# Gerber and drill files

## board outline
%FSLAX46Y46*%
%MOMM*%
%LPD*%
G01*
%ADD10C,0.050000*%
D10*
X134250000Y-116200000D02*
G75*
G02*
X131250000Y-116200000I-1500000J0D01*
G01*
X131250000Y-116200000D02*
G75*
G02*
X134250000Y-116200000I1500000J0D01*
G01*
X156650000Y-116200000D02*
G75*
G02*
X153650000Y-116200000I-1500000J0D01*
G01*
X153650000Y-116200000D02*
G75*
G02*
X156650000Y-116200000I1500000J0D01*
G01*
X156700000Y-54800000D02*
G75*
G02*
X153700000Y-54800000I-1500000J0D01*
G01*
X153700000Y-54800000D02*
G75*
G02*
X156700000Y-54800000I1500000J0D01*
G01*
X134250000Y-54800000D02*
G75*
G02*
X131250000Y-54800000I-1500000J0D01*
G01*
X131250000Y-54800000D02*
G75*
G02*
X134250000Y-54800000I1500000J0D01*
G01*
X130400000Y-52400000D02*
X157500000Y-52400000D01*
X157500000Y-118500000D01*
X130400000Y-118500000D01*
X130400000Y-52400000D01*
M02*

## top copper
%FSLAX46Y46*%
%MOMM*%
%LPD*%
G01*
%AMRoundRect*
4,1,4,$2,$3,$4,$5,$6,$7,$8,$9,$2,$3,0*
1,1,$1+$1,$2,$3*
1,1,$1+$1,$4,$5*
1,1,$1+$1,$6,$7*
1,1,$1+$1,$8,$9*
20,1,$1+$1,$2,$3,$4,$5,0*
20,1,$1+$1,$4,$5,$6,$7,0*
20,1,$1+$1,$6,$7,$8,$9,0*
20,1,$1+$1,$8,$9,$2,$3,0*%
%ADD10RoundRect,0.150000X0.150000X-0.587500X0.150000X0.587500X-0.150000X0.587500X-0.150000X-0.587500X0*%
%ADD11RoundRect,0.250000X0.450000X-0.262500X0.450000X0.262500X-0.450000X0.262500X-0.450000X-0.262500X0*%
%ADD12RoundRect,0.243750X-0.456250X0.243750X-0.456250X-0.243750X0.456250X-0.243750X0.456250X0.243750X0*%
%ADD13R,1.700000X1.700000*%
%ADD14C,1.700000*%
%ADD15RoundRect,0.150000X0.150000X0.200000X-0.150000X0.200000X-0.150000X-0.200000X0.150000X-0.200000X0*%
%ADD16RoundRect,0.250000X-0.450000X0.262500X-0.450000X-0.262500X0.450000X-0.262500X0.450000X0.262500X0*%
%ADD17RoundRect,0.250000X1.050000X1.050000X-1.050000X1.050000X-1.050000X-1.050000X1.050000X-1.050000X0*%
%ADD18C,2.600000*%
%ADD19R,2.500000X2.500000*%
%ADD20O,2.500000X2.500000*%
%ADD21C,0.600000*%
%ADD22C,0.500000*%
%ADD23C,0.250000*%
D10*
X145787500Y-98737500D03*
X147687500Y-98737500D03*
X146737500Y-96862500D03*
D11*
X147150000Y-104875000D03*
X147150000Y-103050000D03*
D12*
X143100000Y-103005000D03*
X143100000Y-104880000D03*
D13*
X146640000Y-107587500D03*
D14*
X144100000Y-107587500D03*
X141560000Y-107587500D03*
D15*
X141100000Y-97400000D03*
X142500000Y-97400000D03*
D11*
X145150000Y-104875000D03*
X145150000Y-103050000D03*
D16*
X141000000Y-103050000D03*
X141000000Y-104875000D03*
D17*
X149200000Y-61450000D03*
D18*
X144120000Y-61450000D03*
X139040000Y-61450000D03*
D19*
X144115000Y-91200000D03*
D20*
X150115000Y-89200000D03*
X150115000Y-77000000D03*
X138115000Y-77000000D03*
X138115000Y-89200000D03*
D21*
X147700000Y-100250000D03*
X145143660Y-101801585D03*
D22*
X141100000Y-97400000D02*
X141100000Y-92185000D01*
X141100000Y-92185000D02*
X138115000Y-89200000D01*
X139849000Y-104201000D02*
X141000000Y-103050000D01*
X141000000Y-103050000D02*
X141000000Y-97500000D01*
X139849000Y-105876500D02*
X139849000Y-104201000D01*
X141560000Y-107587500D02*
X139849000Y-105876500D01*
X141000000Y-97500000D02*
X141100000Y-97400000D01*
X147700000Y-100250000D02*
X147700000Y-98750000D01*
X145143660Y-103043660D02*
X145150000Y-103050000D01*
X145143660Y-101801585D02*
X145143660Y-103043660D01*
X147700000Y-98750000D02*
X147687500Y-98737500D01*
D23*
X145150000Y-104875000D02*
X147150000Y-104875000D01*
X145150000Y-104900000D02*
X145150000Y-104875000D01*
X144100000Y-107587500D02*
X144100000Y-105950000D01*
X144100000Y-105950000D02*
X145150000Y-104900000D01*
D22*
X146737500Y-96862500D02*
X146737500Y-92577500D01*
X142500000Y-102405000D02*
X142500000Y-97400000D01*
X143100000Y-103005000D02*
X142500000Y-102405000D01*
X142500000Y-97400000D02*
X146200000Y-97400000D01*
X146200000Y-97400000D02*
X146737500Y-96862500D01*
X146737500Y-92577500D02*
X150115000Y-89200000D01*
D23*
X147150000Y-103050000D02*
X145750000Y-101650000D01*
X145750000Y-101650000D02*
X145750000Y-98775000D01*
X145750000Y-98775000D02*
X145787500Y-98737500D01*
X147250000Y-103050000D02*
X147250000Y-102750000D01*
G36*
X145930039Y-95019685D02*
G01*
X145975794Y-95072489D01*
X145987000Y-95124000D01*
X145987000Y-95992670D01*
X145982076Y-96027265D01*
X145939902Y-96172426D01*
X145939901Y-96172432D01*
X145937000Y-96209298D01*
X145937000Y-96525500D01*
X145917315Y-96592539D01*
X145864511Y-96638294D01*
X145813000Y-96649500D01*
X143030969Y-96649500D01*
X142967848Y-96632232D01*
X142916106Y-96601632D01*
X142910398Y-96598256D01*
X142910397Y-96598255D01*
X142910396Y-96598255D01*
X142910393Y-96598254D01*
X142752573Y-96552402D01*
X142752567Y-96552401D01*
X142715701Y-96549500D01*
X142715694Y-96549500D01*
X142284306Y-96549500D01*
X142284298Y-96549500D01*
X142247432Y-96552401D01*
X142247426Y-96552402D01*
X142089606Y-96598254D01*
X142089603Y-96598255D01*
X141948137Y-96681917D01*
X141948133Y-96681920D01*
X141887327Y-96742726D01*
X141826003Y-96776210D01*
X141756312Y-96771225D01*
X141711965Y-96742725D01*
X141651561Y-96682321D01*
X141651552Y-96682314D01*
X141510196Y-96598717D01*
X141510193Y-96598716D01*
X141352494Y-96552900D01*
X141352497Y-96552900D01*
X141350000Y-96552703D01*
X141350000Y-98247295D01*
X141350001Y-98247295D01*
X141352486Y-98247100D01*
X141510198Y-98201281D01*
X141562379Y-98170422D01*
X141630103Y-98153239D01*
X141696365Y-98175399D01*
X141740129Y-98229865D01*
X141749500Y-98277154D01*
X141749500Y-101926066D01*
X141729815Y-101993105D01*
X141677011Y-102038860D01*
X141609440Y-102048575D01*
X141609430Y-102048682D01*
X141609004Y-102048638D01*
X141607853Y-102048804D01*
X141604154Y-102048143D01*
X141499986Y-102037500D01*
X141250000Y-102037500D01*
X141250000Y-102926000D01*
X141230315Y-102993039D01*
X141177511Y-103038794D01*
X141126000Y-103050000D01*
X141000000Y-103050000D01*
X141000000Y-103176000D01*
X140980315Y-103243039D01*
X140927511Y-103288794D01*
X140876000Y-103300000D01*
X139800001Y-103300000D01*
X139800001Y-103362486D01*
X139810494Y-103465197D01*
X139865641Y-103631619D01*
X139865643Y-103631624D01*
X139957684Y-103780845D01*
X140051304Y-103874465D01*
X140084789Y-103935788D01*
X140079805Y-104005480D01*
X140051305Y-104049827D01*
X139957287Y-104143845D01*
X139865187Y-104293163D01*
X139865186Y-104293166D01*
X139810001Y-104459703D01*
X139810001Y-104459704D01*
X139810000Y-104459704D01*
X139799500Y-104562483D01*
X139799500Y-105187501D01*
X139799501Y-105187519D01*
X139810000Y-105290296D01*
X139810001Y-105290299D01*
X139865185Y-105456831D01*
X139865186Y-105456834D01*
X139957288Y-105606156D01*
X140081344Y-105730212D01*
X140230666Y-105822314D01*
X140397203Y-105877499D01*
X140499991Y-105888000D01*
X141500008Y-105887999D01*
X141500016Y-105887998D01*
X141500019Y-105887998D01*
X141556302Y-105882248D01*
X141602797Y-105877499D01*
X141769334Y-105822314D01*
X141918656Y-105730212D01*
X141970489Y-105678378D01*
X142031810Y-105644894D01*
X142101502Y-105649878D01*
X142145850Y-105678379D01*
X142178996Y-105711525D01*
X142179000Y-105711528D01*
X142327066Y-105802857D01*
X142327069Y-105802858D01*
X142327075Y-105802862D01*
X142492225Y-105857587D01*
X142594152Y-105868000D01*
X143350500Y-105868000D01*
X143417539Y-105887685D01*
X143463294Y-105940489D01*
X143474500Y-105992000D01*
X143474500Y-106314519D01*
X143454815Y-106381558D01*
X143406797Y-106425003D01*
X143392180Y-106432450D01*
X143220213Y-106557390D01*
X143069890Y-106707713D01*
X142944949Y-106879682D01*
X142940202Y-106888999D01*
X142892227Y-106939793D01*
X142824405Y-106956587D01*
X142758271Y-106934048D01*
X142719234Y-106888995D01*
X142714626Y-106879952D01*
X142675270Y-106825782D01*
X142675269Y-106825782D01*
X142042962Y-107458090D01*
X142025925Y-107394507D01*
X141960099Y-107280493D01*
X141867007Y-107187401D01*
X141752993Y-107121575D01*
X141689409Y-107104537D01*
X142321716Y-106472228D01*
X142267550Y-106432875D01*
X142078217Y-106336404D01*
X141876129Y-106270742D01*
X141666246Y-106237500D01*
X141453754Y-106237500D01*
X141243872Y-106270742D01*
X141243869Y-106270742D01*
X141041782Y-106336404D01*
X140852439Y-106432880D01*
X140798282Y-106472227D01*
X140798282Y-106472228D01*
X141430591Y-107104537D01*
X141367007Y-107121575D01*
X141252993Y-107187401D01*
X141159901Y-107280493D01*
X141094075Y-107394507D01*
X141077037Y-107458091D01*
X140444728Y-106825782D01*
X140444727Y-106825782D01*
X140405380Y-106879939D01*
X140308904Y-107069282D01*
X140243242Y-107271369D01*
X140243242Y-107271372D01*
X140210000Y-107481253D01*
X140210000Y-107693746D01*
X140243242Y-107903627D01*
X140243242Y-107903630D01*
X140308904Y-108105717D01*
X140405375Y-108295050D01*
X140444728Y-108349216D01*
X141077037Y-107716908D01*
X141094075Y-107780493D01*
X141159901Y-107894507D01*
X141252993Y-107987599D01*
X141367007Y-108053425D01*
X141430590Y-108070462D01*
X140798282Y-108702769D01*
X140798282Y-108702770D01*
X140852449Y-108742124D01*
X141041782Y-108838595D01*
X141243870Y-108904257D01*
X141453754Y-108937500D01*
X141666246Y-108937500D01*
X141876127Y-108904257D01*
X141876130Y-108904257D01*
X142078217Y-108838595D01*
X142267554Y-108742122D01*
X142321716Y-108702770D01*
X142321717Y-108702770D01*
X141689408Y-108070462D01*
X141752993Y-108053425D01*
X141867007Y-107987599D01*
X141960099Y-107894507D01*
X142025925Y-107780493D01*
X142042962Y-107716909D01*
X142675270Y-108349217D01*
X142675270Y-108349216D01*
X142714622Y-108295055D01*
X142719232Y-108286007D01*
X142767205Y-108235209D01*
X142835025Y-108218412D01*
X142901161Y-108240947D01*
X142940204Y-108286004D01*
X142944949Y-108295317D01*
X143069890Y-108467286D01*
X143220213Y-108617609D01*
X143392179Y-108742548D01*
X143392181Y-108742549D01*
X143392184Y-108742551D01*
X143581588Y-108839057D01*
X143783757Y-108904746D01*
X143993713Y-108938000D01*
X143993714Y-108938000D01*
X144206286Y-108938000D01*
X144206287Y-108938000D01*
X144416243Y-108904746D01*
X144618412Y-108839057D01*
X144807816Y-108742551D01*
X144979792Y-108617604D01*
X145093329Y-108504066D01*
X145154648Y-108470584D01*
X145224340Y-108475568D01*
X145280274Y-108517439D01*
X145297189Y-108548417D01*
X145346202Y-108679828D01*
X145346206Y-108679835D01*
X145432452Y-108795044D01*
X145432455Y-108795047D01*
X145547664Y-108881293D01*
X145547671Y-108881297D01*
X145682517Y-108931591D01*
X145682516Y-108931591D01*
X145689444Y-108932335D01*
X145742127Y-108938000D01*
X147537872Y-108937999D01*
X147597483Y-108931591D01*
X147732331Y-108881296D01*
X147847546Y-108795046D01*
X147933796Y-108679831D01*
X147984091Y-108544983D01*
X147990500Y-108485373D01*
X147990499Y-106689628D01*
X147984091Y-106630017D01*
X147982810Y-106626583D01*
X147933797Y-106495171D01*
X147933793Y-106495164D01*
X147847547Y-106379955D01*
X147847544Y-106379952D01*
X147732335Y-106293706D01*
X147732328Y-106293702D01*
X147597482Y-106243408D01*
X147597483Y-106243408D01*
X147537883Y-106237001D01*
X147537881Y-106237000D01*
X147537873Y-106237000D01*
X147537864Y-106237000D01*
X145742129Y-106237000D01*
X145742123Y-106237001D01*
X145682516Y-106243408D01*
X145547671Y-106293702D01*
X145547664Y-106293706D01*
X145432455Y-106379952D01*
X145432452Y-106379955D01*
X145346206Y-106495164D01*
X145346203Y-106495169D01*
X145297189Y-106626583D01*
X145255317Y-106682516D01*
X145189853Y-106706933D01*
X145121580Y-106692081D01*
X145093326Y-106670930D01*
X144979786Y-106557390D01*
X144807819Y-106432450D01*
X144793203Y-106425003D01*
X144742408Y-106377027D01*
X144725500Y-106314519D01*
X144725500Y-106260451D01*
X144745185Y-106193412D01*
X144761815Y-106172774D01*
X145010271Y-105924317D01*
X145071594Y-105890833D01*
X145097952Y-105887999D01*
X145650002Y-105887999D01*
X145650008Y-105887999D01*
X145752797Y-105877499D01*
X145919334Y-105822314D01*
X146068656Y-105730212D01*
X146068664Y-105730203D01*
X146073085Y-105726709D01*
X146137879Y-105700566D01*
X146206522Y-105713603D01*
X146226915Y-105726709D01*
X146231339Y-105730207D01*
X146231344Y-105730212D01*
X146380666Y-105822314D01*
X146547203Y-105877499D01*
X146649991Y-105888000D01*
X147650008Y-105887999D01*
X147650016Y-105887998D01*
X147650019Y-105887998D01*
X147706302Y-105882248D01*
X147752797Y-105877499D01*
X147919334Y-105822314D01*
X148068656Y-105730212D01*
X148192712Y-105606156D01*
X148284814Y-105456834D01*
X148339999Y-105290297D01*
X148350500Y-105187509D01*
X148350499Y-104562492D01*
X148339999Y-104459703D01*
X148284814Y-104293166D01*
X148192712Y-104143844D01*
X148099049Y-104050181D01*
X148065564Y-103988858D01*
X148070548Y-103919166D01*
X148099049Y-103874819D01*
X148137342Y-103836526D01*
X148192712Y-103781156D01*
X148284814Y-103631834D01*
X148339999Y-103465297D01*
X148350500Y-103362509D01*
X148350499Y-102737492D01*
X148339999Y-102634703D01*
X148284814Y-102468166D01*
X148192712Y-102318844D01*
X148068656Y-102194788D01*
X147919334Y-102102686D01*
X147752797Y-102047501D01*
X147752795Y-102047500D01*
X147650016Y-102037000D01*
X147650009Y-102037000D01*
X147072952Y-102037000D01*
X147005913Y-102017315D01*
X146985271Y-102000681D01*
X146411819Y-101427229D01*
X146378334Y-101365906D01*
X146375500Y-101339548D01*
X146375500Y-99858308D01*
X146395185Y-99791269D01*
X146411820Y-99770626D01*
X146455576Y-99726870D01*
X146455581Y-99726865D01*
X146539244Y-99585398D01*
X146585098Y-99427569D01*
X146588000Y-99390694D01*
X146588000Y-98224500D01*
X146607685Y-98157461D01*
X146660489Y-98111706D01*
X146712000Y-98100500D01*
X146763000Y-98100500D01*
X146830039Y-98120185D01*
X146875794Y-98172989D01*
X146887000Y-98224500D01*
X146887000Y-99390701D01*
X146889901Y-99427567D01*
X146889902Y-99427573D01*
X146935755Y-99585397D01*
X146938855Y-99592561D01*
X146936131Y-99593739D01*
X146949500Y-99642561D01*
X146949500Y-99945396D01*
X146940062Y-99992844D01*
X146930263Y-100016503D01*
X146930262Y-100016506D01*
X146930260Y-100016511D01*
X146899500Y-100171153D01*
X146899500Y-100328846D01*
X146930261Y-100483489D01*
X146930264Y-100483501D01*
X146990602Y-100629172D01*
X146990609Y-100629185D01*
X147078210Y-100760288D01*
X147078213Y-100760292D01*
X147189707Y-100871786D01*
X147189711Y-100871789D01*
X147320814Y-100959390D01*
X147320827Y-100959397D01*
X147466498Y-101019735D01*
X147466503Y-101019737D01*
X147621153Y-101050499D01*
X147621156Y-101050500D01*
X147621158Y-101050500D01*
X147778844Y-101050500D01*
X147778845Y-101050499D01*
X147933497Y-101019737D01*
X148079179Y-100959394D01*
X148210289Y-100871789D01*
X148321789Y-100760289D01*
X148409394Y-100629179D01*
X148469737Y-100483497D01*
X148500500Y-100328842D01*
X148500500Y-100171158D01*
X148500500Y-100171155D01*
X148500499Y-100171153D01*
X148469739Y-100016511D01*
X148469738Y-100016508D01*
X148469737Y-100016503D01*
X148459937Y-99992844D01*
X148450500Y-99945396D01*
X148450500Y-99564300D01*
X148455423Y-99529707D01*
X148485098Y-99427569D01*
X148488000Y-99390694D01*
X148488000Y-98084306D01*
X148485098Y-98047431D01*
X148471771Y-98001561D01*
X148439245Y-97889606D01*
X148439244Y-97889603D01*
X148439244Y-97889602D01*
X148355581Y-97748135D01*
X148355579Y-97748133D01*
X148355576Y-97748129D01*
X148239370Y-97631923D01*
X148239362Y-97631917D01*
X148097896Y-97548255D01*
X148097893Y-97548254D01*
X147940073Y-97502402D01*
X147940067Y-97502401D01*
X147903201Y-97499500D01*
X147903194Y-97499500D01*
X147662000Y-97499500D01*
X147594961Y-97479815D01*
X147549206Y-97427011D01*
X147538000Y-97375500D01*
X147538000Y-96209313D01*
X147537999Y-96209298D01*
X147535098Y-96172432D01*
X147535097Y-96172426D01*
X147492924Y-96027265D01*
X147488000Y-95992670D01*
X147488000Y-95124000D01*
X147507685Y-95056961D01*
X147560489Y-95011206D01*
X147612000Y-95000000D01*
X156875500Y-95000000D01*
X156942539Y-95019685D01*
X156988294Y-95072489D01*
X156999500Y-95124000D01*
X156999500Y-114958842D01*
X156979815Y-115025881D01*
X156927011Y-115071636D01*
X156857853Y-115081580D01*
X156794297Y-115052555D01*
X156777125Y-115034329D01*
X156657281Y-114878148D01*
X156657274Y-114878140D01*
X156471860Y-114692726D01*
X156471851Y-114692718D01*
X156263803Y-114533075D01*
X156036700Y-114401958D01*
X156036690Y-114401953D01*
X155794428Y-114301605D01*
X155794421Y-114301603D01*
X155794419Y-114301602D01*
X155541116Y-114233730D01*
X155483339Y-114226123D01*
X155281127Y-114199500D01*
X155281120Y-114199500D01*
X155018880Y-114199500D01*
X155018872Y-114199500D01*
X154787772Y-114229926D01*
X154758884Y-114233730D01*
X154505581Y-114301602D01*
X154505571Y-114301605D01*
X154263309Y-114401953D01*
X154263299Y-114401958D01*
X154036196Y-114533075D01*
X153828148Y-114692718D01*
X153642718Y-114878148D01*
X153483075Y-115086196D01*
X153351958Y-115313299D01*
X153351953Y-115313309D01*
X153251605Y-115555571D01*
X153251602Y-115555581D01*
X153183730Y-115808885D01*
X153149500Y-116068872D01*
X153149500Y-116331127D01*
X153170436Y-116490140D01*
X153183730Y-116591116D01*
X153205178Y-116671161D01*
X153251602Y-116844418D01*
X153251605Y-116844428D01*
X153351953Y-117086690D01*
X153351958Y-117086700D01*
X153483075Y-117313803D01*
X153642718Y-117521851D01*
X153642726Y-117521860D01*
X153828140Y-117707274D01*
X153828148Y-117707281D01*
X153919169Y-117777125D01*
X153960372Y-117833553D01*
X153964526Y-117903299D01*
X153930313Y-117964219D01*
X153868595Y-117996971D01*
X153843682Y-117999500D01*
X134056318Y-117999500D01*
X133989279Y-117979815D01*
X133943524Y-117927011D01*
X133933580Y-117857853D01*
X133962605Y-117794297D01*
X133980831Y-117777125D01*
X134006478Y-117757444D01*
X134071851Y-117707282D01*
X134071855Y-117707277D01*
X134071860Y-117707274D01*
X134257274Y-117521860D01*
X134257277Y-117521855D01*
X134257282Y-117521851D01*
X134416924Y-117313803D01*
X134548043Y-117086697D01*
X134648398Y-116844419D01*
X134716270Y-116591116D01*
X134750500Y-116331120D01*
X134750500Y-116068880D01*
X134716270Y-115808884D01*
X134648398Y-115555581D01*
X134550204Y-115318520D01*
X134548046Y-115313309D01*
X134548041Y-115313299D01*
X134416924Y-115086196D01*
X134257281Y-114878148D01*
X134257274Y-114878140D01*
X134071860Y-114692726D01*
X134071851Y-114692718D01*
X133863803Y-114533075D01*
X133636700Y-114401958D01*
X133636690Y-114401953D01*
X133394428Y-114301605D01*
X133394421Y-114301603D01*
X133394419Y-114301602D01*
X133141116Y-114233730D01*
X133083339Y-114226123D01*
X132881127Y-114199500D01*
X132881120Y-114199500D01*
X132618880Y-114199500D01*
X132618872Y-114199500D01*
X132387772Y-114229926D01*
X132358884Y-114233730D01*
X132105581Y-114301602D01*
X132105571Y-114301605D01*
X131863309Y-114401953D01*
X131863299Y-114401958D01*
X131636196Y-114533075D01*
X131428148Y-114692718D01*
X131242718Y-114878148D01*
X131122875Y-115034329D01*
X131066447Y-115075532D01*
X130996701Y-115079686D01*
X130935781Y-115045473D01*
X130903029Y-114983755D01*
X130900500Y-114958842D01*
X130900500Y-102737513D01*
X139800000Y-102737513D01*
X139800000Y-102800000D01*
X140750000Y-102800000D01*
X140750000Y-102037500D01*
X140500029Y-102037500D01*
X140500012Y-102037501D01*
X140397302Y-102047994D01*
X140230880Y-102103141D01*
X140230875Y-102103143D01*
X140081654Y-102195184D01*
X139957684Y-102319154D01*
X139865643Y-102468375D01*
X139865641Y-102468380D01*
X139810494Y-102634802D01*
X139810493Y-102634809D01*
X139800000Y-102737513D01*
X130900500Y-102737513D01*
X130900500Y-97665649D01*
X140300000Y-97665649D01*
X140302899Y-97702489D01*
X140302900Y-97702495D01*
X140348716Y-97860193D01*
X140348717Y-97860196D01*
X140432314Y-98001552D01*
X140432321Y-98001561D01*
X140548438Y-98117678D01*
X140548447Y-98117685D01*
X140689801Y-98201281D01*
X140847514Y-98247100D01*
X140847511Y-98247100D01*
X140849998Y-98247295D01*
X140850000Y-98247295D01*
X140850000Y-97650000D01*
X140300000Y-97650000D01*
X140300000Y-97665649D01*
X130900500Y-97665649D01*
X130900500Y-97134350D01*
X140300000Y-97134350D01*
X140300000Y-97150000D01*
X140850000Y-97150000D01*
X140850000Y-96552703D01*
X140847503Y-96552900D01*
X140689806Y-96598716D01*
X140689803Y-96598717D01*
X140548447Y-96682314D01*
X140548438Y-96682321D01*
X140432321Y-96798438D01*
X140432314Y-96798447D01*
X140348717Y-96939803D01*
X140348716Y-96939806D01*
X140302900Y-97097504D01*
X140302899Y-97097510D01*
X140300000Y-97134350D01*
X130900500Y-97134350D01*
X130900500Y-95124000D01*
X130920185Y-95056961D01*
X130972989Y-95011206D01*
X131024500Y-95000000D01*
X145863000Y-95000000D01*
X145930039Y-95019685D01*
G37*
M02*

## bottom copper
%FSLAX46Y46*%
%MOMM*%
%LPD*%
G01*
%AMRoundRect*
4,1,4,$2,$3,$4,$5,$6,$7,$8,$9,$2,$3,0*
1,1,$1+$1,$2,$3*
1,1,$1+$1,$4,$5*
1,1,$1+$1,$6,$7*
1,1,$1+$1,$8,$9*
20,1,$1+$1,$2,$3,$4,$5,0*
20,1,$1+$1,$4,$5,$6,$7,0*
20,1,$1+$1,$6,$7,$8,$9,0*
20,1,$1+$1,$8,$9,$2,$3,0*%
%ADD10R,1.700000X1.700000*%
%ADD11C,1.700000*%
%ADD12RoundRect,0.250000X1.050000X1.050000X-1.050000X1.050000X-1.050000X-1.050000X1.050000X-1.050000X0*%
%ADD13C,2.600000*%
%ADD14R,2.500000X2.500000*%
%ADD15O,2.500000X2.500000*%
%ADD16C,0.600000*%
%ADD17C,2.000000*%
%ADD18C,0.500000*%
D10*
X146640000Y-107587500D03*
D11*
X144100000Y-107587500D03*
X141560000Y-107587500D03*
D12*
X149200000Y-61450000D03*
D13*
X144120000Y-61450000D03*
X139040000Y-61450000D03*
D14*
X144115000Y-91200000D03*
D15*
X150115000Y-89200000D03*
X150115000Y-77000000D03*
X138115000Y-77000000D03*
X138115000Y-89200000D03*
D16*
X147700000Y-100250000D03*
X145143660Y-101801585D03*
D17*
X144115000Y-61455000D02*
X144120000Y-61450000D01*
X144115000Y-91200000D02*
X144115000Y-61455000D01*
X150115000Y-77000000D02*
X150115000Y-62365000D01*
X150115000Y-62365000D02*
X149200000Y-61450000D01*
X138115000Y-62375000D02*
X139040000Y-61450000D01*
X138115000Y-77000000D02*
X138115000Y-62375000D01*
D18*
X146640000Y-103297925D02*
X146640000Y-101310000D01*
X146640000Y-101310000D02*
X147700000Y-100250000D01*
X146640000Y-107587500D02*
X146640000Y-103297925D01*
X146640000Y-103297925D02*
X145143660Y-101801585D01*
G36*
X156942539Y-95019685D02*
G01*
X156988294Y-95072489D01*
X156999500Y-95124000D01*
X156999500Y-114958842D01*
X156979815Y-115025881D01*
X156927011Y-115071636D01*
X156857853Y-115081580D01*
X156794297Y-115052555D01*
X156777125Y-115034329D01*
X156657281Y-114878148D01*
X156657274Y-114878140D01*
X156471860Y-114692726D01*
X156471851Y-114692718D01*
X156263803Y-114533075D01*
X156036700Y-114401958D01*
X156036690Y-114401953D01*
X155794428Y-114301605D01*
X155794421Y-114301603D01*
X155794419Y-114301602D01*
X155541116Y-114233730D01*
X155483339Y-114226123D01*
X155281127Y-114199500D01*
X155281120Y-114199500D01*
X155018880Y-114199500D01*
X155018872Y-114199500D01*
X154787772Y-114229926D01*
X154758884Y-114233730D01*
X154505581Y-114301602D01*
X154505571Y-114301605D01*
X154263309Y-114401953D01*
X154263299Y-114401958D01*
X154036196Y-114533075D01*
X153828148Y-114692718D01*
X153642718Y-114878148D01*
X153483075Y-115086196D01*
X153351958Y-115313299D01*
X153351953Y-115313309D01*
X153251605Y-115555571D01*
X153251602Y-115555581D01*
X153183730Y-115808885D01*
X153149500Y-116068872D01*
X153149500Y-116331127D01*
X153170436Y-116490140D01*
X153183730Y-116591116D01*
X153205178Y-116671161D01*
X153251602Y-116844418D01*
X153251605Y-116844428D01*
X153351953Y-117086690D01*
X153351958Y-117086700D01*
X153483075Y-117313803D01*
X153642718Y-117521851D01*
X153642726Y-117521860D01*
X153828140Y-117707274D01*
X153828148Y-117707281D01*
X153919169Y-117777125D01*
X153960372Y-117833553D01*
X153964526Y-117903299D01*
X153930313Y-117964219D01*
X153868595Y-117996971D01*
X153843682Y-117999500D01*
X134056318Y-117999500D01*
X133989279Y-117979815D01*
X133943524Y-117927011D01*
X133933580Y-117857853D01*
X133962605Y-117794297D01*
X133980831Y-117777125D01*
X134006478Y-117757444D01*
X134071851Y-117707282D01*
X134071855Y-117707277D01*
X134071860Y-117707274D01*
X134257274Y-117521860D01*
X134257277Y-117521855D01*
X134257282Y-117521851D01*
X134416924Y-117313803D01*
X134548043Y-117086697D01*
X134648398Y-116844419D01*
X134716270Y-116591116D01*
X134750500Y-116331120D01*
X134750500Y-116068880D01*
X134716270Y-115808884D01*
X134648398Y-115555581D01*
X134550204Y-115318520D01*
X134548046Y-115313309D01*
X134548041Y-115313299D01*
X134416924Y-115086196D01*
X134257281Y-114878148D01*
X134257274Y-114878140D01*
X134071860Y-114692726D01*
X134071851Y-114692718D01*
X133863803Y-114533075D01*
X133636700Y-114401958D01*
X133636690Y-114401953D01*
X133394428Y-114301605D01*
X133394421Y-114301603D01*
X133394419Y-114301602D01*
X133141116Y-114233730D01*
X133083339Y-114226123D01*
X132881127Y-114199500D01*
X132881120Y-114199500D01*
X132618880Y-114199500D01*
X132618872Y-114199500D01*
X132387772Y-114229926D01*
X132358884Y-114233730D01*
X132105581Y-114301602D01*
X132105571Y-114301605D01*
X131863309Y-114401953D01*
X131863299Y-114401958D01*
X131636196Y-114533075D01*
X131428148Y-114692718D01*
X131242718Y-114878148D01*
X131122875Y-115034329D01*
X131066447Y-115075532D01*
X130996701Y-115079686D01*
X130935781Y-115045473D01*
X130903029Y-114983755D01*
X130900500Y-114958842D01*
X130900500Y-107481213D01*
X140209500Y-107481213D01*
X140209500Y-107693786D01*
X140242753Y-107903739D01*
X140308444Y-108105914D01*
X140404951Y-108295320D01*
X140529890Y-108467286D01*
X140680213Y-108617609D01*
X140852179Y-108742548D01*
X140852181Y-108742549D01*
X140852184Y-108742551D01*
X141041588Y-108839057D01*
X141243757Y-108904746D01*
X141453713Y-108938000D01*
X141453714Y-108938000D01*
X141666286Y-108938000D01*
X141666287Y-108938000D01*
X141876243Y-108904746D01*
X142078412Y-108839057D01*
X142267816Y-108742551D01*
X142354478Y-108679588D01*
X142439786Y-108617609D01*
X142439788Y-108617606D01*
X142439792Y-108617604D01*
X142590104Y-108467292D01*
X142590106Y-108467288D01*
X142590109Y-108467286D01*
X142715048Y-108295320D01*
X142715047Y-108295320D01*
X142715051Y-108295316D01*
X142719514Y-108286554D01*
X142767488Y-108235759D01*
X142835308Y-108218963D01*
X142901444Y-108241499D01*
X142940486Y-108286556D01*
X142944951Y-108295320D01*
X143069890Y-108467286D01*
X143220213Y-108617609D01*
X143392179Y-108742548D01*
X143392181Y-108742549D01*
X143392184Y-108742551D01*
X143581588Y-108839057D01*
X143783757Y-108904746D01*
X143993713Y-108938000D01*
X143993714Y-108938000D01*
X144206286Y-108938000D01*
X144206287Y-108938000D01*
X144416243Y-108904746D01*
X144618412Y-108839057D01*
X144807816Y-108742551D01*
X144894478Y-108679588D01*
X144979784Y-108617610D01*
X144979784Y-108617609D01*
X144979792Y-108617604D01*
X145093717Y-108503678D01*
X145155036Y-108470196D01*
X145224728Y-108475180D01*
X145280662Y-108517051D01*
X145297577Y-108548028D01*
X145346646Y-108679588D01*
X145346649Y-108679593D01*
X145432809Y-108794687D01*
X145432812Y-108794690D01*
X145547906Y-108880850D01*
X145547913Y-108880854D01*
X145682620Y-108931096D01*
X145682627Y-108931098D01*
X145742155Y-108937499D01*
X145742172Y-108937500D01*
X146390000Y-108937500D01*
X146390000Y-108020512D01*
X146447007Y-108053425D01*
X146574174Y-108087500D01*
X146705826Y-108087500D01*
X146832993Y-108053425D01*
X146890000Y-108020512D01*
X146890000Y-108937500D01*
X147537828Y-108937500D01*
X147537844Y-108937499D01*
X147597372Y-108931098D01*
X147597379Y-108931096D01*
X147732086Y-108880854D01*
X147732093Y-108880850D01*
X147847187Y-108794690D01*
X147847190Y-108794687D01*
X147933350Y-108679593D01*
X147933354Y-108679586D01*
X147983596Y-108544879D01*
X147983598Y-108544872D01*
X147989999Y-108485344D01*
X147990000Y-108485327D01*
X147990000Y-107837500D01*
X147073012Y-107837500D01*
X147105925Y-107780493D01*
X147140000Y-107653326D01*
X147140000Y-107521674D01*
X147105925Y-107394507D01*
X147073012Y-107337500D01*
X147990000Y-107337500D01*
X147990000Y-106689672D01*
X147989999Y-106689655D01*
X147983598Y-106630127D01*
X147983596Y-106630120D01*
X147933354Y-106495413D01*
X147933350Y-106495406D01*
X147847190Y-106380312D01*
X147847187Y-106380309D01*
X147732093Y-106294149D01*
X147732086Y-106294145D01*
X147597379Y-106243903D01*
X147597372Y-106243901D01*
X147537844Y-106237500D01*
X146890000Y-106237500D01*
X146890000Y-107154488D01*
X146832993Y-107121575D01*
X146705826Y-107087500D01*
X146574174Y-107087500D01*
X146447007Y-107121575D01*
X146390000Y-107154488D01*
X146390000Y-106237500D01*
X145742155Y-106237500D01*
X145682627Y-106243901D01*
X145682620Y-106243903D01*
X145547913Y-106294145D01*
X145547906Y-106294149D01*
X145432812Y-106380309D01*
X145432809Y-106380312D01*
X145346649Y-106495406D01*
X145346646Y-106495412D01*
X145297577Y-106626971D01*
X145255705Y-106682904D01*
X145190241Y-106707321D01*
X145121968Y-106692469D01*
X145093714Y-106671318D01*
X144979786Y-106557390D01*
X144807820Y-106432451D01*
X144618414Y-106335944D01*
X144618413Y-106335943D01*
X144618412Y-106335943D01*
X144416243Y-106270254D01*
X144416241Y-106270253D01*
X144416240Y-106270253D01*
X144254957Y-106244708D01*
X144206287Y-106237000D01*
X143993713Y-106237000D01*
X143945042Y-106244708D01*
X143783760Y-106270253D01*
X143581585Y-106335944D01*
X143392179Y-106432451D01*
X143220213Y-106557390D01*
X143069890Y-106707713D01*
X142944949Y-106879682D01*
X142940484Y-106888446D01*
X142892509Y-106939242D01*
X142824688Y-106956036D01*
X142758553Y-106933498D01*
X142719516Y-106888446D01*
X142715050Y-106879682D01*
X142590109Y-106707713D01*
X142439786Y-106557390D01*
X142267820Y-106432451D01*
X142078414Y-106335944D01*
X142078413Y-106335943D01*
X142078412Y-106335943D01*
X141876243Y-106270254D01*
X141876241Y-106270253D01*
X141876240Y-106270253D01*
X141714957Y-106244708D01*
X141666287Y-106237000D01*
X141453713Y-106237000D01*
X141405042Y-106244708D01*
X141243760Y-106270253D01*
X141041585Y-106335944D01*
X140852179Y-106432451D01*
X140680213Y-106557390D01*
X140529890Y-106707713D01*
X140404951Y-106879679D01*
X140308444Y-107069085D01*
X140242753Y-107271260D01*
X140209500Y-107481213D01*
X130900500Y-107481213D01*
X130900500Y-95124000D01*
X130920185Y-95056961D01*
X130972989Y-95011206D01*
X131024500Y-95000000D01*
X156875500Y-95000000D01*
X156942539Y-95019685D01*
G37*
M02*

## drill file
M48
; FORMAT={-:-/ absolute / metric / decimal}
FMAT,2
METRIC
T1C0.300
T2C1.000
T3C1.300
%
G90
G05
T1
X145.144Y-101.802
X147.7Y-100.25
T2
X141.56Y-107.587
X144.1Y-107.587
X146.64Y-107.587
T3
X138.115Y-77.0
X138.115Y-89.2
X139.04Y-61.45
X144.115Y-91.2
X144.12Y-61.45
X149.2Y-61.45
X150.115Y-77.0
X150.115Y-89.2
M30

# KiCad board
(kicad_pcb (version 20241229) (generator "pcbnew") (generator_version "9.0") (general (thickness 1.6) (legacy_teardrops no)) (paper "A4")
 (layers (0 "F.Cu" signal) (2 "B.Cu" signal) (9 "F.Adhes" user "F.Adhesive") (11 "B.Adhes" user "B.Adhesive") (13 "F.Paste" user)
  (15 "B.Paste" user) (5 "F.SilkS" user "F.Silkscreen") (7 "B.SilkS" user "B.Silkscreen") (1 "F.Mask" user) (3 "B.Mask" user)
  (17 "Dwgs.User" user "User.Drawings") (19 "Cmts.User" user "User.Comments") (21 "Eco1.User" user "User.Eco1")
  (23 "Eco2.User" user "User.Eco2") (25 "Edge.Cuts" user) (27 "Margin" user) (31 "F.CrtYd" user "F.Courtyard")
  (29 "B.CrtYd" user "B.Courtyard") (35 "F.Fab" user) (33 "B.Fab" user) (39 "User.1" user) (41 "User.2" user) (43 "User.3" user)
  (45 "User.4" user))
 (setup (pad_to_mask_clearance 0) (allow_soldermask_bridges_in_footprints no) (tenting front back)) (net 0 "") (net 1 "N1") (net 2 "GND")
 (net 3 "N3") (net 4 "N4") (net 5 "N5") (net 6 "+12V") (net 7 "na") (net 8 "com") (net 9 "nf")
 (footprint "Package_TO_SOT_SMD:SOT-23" (layer "F.Cu") (at 146.7375 97.8 90)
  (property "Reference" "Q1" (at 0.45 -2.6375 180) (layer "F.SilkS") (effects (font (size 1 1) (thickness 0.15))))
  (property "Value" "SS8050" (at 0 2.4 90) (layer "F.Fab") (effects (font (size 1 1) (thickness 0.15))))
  (pad "1" smd roundrect (at -0.9375 -0.95 90) (size 1.475 0.6) (layers "F.Cu" "F.Mask" "F.Paste") (roundrect_rratio 0.25) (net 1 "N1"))
  (pad "2" smd roundrect (at -0.9375 0.95 90) (size 1.475 0.6) (layers "F.Cu" "F.Mask" "F.Paste") (roundrect_rratio 0.25) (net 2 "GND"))
  (pad "3" smd roundrect (at 0.9375 0 90) (size 1.475 0.6) (layers "F.Cu" "F.Mask" "F.Paste") (roundrect_rratio 0.25) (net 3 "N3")))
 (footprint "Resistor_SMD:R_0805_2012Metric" (layer "F.Cu") (at 147.15 103.9625 90)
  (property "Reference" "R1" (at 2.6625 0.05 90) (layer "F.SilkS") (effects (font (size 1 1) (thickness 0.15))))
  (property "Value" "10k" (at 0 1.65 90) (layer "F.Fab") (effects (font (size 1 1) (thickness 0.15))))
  (pad "1" smd roundrect (at -0.9125 0 90) (size 1.025 1.4) (layers "F.Cu" "F.Mask" "F.Paste") (roundrect_rratio 0.243902) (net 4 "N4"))
  (pad "2" smd roundrect (at 0.9125 0 90) (size 1.025 1.4) (layers "F.Cu" "F.Mask" "F.Paste") (roundrect_rratio 0.243902) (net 1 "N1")))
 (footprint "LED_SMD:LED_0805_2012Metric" (layer "F.Cu") (at 143.1 103.9425 -90)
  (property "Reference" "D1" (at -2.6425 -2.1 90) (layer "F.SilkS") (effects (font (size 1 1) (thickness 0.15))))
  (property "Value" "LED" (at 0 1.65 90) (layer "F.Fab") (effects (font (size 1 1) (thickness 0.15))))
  (pad "1" smd roundrect (at -0.9375 0 270) (size 0.975 1.4) (layers "F.Cu" "F.Mask" "F.Paste") (roundrect_rratio 0.25) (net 3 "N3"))
  (pad "2" smd roundrect (at 0.9375 0 270) (size 0.975 1.4) (layers "F.Cu" "F.Mask" "F.Paste") (roundrect_rratio 0.25) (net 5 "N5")))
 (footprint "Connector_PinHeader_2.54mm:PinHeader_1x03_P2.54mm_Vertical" (layer "F.Cu") (at 146.64 107.5875 -90)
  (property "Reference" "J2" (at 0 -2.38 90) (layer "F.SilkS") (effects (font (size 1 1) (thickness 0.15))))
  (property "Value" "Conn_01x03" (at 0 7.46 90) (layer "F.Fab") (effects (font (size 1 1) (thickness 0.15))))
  (pad "1" thru_hole rect (at 0 0 270) (size 1.7 1.7) (drill 1) (layers "*.Cu" "*.Mask") (remove_unused_layers no) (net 2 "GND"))
  (pad "2" thru_hole circle (at 0 2.54 270) (size 1.7 1.7) (drill 1) (layers "*.Cu" "*.Mask") (remove_unused_layers no) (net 4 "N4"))
  (pad "3" thru_hole circle (at 0 5.08 270) (size 1.7 1.7) (drill 1) (layers "*.Cu" "*.Mask") (remove_unused_layers no) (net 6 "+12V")))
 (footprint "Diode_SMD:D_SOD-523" (layer "F.Cu") (at 141.8 97.4)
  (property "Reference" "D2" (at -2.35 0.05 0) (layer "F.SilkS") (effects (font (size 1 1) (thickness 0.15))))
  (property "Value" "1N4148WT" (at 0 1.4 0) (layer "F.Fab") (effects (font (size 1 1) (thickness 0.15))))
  (pad "1" smd roundrect (at -0.7 0 180) (size 0.6 0.7) (layers "F.Cu" "F.Mask" "F.Paste") (roundrect_rratio 0.25) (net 6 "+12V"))
  (pad "2" smd roundrect (at 0.7 0 180) (size 0.6 0.7) (layers "F.Cu" "F.Mask" "F.Paste") (roundrect_rratio 0.25) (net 3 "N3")))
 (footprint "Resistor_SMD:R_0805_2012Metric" (layer "F.Cu") (at 145.15 103.9625 90)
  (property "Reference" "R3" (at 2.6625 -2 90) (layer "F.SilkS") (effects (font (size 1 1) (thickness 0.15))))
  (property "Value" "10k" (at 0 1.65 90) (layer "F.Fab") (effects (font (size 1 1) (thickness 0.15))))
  (pad "1" smd roundrect (at -0.9125 0 90) (size 1.025 1.4) (layers "F.Cu" "F.Mask" "F.Paste") (roundrect_rratio 0.243902) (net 4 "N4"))
  (pad "2" smd roundrect (at 0.9125 0 90) (size 1.025 1.4) (layers "F.Cu" "F.Mask" "F.Paste") (roundrect_rratio 0.243902) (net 2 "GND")))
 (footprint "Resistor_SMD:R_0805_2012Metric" (layer "F.Cu") (at 141 103.9625 -90)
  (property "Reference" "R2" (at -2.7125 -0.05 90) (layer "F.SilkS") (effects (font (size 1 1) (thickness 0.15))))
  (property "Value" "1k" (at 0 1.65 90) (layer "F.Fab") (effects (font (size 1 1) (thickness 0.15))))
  (pad "1" smd roundrect (at -0.9125 0 270) (size 1.025 1.4) (layers "F.Cu" "F.Mask" "F.Paste") (roundrect_rratio 0.243902) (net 6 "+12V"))
  (pad "2" smd roundrect (at 0.9125 0 270) (size 1.025 1.4) (layers "F.Cu" "F.Mask" "F.Paste") (roundrect_rratio 0.243902) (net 5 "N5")))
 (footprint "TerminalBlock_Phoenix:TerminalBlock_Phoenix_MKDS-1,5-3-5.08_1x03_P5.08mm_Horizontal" (layer "F.Cu") (at 149.2 61.45 180)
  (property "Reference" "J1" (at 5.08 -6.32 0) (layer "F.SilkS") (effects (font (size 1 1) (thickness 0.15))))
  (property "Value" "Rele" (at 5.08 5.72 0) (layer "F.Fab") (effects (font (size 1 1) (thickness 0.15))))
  (pad "1" thru_hole roundrect (at 0 0 180) (size 2.6 2.6) (drill 1.3) (layers "*.Cu" "*.Mask") (remove_unused_layers no)
   (roundrect_rratio 0.096154) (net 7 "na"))
  (pad "2" thru_hole circle (at 5.08 0 180) (size 2.6 2.6) (drill 1.3) (layers "*.Cu" "*.Mask") (remove_unused_layers no) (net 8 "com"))
  (pad "3" thru_hole circle (at 10.16 0 180) (size 2.6 2.6) (drill 1.3) (layers "*.Cu" "*.Mask") (remove_unused_layers no) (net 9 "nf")))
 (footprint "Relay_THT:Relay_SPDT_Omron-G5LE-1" (layer "F.Cu") (at 144.115 91.2 180)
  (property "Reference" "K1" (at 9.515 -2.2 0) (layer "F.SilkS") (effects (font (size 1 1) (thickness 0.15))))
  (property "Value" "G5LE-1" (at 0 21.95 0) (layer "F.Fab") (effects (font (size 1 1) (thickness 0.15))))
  (pad "1" thru_hole rect (at 0 0 180) (size 2.5 2.5) (drill 1.3) (layers "*.Cu" "*.Mask") (remove_unused_layers no) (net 8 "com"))
  (pad "2" thru_hole oval (at -6 2 180) (size 2.5 2.5) (drill 1.3) (layers "*.Cu" "*.Mask") (remove_unused_layers no) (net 3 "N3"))
  (pad "3" thru_hole oval (at -6 14.2 180) (size 2.5 2.5) (drill 1.3) (layers "*.Cu" "*.Mask") (remove_unused_layers no) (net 7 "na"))
  (pad "4" thru_hole oval (at 6 14.2 180) (size 2.5 2.5) (drill 1.3) (layers "*.Cu" "*.Mask") (remove_unused_layers no) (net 9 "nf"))
  (pad "5" thru_hole oval (at 6 2 180) (size 2.5 2.5) (drill 1.3) (layers "*.Cu" "*.Mask") (remove_unused_layers no) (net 6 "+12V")))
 (gr_circle (center 132.75 116.2) (end 131.25 116.2) (stroke (width 0.05) (type default)) (fill no) (layer "Edge.Cuts"))
 (gr_circle (center 155.15 116.2) (end 153.65 116.2) (stroke (width 0.05) (type default)) (fill no) (layer "Edge.Cuts"))
 (gr_circle (center 155.2 54.8) (end 153.7 54.8) (stroke (width 0.05) (type default)) (fill no) (layer "Edge.Cuts"))
 (gr_circle (center 132.75 54.8) (end 131.25 54.8) (stroke (width 0.05) (type default)) (fill no) (layer "Edge.Cuts"))
 (gr_rect (start 130.4 52.4) (end 157.5 118.5) (stroke (width 0.05) (type default)) (fill no) (layer "Edge.Cuts"))
 (segment (start 141.1 97.4) (end 141.1 92.185) (width 0.5) (layer "F.Cu") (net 6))
 (segment (start 141.1 92.185) (end 138.115 89.2) (width 0.5) (layer "F.Cu") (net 6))
 (segment (start 139.849 104.201) (end 141 103.05) (width 0.5) (layer "F.Cu") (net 6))
 (segment (start 141 103.05) (end 141 97.5) (width 0.5) (layer "F.Cu") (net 6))
 (segment (start 139.849 105.8765) (end 139.849 104.201) (width 0.5) (layer "F.Cu") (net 6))
 (segment (start 141.56 107.5875) (end 139.849 105.8765) (width 0.5) (layer "F.Cu") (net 6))
 (segment (start 141 97.5) (end 141.1 97.4) (width 0.5) (layer "F.Cu") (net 6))
 (segment (start 144.115 61.455) (end 144.12 61.45) (width 2) (layer "B.Cu") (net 8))
 (segment (start 144.115 91.2) (end 144.115 61.455) (width 2) (layer "B.Cu") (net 8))
 (segment (start 150.115 77) (end 150.115 62.365) (width 2) (layer "B.Cu") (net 7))
 (segment (start 150.115 62.365) (end 149.2 61.45) (width 2) (layer "B.Cu") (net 7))
 (segment (start 138.115 62.375) (end 139.04 61.45) (width 2) (layer "B.Cu") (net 9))
 (segment (start 138.115 77) (end 138.115 62.375) (width 2) (layer "B.Cu") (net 9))
 (segment (start 147.7 100.25) (end 147.7 98.75) (width 0.5) (layer "F.Cu") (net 2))
 (segment (start 145.14366 103.04366) (end 145.15 103.05) (width 0.5) (layer "F.Cu") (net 2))
 (segment (start 145.14366 101.801585) (end 145.14366 103.04366) (width 0.5) (layer "F.Cu") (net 2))
 (segment (start 147.7 98.75) (end 147.6875 98.7375) (width 0.5) (layer "F.Cu") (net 2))
 (via (at 147.7 100.25) (size 0.6) (drill 0.3) (layers "F.Cu" "B.Cu") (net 2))
 (via (at 145.14366 101.801585) (size 0.6) (drill 0.3) (layers "F.Cu" "B.Cu") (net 2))
 (segment (start 146.64 103.297925) (end 146.64 101.31) (width 0.5) (layer "B.Cu") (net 2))
 (segment (start 146.64 101.31) (end 147.7 100.25) (width 0.5) (layer "B.Cu") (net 2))
 (segment (start 146.64 107.5875) (end 146.64 103.297925) (width 0.5) (layer "B.Cu") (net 2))
 (segment (start 146.64 103.297925) (end 145.14366 101.801585) (width 0.5) (layer "B.Cu") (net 2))
 (segment (start 145.15 104.875) (end 147.15 104.875) (width 0.25) (layer "F.Cu") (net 4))
 (segment (start 145.15 104.9) (end 145.15 104.875) (width 0.25) (layer "F.Cu") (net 4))
 (segment (start 144.1 107.5875) (end 144.1 105.95) (width 0.25) (layer "F.Cu") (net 4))
 (segment (start 144.1 105.95) (end 145.15 104.9) (width 0.25) (layer "F.Cu") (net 4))
 (segment (start 146.7375 96.8625) (end 146.7375 92.5775) (width 0.5) (layer "F.Cu") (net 3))
 (segment (start 142.5 102.405) (end 142.5 97.4) (width 0.5) (layer "F.Cu") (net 3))
 (segment (start 143.1 103.005) (end 142.5 102.405) (width 0.5) (layer "F.Cu") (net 3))
 (segment (start 142.5 97.4) (end 146.2 97.4) (width 0.5) (layer "F.Cu") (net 3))
 (segment (start 146.2 97.4) (end 146.7375 96.8625) (width 0.5) (layer "F.Cu") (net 3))
 (segment (start 146.7375 92.5775) (end 150.115 89.2) (width 0.5) (layer "F.Cu") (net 3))
 (segment (start 147.15 103.05) (end 145.75 101.65) (width 0.25) (layer "F.Cu") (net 1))
 (segment (start 145.75 101.65) (end 145.75 98.775) (width 0.25) (layer "F.Cu") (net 1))
 (segment (start 145.75 98.775) (end 145.7875 98.7375) (width 0.25) (layer "F.Cu") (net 1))
 (segment (start 147.25 103.05) (end 147.25 102.75) (width 0.25) (layer "F.Cu") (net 1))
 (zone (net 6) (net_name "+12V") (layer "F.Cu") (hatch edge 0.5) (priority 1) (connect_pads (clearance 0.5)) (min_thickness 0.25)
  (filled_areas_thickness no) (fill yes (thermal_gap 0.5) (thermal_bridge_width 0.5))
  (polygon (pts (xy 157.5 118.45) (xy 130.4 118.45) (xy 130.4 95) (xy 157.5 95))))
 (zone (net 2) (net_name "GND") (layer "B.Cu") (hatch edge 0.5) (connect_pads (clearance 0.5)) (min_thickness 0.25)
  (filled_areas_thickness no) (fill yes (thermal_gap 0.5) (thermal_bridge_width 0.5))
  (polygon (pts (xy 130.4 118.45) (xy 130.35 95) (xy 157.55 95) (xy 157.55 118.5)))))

